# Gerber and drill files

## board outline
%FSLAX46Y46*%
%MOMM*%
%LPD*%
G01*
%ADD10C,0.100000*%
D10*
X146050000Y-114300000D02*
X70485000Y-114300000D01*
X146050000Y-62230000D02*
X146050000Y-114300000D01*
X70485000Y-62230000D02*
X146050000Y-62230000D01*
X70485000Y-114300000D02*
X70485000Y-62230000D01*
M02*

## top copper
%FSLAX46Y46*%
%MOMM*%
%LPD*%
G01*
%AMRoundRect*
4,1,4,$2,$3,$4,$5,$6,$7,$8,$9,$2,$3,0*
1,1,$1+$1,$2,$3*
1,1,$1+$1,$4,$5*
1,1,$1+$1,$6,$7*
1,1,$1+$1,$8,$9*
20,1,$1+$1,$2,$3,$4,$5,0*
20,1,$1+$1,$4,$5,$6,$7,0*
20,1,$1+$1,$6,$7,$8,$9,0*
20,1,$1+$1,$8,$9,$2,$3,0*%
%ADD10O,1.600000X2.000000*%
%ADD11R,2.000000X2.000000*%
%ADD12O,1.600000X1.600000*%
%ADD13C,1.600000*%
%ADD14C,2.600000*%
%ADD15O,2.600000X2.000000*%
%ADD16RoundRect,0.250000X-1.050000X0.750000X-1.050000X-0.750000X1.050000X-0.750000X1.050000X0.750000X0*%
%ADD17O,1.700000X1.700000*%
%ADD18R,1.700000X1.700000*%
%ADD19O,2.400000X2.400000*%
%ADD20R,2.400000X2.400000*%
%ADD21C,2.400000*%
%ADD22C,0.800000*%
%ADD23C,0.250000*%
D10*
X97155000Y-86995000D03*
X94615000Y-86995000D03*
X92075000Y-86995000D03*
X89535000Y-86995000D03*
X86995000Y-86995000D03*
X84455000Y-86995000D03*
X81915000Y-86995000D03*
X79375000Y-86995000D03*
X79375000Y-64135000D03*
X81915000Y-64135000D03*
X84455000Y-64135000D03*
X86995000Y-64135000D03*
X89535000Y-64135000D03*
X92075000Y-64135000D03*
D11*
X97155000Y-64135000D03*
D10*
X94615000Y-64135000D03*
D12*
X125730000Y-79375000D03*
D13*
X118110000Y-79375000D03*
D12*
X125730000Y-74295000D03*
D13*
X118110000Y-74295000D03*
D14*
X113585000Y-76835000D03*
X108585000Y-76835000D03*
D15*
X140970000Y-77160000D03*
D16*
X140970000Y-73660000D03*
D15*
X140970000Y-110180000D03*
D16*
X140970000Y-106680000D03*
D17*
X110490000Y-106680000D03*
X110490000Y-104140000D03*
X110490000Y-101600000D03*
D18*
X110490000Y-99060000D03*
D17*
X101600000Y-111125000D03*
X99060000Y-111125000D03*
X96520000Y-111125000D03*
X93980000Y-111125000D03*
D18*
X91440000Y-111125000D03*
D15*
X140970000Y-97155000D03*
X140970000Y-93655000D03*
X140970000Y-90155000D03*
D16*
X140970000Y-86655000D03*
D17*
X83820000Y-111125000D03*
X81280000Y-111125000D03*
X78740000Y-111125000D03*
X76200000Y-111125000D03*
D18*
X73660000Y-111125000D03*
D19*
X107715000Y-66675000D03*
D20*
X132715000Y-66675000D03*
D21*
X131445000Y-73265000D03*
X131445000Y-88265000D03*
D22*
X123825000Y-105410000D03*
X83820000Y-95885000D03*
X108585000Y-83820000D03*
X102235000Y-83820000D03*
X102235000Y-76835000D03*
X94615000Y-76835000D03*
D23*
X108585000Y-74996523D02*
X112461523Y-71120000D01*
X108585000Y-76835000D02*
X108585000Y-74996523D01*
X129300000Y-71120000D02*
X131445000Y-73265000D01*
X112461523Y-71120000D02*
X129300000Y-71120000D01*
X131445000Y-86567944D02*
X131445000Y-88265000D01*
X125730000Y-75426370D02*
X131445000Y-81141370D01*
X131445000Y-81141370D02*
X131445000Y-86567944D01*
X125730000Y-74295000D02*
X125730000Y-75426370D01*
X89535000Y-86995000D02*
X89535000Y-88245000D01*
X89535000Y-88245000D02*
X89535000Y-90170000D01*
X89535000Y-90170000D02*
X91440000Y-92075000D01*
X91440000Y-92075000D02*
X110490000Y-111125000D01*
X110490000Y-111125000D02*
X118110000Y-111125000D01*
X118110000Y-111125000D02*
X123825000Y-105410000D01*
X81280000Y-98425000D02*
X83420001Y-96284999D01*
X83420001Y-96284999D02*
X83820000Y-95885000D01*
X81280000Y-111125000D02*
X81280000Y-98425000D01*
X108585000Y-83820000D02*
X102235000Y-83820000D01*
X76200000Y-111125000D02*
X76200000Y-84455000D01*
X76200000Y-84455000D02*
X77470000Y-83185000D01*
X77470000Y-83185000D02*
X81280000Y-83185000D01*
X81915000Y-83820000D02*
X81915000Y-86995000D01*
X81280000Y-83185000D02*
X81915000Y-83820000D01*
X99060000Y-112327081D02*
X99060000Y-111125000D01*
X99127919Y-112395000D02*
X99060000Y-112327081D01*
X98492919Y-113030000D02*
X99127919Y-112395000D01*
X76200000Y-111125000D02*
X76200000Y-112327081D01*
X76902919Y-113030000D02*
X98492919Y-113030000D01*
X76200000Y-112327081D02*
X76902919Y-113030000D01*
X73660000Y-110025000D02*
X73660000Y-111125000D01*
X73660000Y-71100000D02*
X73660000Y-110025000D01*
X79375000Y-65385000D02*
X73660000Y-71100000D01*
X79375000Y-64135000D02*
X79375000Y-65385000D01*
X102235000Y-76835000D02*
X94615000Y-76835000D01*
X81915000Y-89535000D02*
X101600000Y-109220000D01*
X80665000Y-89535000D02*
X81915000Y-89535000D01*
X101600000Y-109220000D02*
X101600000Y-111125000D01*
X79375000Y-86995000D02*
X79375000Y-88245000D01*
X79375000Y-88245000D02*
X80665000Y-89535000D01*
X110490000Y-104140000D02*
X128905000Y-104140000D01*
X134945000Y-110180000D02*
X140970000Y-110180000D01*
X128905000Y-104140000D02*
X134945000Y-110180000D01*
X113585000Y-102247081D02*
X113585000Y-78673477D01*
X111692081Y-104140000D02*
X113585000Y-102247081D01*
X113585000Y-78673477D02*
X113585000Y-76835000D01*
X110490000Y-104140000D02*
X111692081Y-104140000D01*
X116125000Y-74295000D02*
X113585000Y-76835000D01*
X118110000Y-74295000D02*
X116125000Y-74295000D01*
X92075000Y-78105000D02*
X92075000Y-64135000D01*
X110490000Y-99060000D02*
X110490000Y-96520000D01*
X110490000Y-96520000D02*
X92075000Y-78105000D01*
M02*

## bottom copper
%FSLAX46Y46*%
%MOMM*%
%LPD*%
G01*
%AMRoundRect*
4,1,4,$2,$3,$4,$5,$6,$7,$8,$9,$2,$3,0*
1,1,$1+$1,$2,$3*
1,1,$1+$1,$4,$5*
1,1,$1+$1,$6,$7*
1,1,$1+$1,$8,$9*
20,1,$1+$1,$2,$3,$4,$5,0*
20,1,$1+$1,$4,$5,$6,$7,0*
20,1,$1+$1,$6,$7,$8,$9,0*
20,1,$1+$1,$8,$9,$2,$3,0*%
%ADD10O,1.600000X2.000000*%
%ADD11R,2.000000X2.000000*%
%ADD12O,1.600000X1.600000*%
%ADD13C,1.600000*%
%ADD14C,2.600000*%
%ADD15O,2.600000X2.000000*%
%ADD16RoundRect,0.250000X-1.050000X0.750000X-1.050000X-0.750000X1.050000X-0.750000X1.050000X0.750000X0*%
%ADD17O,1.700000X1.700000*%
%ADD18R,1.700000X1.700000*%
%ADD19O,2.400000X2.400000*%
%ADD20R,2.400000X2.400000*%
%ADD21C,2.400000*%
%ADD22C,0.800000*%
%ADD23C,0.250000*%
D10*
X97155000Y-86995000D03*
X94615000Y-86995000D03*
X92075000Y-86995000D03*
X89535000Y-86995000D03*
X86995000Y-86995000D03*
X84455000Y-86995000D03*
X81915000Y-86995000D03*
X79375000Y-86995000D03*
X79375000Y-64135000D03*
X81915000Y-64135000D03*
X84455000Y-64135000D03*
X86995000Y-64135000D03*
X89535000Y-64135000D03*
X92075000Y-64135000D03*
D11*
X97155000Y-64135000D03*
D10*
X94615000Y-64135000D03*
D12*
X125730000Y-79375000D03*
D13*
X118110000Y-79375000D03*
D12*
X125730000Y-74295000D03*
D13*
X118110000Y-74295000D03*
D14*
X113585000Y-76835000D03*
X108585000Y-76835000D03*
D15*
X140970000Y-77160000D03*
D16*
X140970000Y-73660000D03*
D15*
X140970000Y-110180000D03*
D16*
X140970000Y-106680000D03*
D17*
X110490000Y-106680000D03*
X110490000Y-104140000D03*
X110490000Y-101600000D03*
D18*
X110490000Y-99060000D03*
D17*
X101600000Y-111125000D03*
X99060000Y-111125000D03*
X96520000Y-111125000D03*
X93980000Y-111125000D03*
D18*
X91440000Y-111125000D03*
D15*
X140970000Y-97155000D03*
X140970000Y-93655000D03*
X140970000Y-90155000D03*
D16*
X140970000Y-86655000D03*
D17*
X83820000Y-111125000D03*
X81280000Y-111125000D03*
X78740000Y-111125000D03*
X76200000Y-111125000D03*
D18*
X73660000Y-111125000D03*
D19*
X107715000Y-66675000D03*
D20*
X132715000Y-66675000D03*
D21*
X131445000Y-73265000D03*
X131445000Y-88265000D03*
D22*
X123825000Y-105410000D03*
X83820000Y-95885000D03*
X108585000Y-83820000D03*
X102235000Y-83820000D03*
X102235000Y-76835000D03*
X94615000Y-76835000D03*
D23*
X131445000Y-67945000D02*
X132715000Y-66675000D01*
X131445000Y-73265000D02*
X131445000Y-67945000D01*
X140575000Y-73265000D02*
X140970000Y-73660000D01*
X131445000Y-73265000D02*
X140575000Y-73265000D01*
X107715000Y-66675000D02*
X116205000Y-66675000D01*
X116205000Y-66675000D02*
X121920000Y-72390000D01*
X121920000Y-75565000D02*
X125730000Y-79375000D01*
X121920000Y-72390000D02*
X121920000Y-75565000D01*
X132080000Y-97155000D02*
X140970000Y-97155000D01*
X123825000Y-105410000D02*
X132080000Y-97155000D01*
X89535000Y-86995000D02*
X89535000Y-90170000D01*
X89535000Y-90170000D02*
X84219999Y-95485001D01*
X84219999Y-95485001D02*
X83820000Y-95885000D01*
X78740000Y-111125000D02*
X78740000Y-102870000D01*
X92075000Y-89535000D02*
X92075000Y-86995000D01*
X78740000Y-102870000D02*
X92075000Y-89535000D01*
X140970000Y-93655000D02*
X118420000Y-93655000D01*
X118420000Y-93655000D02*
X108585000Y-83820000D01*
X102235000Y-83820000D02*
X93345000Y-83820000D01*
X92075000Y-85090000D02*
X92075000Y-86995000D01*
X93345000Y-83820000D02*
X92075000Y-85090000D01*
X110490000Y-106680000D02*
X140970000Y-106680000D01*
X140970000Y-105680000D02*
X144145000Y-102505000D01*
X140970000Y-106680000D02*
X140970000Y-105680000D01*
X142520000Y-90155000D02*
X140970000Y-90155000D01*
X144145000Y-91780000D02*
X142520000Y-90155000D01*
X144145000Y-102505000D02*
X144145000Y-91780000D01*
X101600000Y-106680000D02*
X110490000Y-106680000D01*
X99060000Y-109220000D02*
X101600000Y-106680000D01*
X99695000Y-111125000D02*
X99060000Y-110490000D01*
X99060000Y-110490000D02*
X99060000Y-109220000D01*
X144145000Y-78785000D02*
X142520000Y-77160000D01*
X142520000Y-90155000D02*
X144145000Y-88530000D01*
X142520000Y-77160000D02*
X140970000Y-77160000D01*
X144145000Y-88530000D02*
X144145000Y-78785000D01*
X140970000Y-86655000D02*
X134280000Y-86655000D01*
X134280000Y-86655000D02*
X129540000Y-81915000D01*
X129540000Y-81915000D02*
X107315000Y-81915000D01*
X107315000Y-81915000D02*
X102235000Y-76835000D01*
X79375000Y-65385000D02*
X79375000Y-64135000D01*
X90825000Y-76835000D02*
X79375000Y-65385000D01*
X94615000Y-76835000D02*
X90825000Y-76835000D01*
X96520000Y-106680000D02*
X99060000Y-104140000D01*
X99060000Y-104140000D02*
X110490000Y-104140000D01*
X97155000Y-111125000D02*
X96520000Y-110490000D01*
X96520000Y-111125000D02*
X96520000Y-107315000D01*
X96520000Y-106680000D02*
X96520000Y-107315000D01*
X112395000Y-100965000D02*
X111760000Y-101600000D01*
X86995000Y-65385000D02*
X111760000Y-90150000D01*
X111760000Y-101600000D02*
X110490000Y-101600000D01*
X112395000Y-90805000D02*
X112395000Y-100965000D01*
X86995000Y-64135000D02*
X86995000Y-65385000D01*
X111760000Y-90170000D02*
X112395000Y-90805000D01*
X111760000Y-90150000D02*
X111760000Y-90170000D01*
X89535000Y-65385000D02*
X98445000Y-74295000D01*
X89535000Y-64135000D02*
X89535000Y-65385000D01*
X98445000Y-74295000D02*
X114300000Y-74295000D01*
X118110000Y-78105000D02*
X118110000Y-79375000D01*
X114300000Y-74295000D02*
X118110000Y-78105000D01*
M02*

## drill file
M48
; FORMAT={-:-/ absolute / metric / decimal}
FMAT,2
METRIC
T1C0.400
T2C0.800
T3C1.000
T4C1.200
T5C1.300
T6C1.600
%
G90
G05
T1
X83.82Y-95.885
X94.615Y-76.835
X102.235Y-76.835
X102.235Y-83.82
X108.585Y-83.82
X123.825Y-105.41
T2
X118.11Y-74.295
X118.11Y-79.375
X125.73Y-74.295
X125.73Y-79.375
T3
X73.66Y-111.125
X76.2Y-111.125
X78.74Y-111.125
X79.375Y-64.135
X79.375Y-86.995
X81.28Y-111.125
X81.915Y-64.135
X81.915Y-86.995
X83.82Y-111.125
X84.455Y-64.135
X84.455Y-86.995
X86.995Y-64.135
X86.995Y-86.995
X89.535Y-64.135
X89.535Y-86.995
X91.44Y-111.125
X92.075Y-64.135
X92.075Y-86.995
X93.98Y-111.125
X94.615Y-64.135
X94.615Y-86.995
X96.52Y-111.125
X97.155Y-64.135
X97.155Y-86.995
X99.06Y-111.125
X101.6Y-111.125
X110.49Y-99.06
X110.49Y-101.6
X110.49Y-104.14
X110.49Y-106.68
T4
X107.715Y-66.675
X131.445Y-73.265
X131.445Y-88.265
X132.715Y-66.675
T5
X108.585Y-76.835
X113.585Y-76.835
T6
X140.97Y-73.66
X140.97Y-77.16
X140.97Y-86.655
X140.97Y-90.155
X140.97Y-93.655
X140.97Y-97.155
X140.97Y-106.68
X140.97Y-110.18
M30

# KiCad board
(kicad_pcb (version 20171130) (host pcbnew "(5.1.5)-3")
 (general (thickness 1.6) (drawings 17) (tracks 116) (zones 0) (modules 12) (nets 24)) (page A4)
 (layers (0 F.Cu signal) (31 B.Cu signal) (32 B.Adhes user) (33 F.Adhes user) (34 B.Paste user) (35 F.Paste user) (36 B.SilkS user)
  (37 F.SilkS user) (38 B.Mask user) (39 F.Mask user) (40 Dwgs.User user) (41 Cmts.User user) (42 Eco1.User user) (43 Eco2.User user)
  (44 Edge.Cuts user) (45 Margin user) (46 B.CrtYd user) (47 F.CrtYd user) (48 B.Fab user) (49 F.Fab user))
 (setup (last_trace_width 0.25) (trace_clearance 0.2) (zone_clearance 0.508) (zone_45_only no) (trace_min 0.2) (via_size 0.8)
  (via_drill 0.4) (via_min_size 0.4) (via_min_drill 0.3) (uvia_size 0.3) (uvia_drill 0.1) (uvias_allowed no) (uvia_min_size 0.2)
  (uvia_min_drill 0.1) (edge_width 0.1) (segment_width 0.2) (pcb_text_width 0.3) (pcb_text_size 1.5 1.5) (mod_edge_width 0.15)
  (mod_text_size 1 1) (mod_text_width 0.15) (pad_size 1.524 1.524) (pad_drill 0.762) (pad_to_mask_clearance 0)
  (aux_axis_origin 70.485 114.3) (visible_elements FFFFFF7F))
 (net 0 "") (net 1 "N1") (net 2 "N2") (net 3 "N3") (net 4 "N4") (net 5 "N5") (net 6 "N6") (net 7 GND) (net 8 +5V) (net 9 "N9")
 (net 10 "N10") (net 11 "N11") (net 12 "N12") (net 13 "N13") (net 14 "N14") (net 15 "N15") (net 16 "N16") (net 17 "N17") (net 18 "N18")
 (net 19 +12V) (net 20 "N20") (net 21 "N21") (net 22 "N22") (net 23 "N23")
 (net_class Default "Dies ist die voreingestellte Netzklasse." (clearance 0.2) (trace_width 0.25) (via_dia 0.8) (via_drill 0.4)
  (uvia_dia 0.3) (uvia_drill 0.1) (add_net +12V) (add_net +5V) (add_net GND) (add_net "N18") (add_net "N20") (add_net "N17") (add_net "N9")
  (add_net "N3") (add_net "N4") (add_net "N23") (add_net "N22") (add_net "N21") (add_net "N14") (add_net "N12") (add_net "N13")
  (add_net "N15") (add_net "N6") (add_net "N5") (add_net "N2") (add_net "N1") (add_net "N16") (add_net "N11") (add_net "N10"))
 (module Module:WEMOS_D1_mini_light (layer F.Cu) (at 97.155 64.135 270)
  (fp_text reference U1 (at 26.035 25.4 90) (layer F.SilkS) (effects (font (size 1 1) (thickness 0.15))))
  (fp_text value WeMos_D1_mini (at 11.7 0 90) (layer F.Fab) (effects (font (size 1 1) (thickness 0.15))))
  (pad 16 thru_hole oval (at 22.86 0 270) (size 2 1.6) (drill 1) (layers *.Cu *.Mask) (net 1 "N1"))
  (pad 15 thru_hole oval (at 22.86 2.54 270) (size 2 1.6) (drill 1) (layers *.Cu *.Mask) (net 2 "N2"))
  (pad 14 thru_hole oval (at 22.86 5.08 270) (size 2 1.6) (drill 1) (layers *.Cu *.Mask) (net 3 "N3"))
  (pad 13 thru_hole oval (at 22.86 7.62 270) (size 2 1.6) (drill 1) (layers *.Cu *.Mask) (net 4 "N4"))
  (pad 12 thru_hole oval (at 22.86 10.16 270) (size 2 1.6) (drill 1) (layers *.Cu *.Mask) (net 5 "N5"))
  (pad 11 thru_hole oval (at 22.86 12.7 270) (size 2 1.6) (drill 1) (layers *.Cu *.Mask) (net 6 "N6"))
  (pad 10 thru_hole oval (at 22.86 15.24 270) (size 2 1.6) (drill 1) (layers *.Cu *.Mask) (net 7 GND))
  (pad 9 thru_hole oval (at 22.86 17.78 270) (size 2 1.6) (drill 1) (layers *.Cu *.Mask) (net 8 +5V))
  (pad 8 thru_hole oval (at 0 17.78 270) (size 2 1.6) (drill 1) (layers *.Cu *.Mask) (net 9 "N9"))
  (pad 7 thru_hole oval (at 0 15.24 270) (size 2 1.6) (drill 1) (layers *.Cu *.Mask) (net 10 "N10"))
  (pad 6 thru_hole oval (at 0 12.7 270) (size 2 1.6) (drill 1) (layers *.Cu *.Mask) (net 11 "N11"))
  (pad 5 thru_hole oval (at 0 10.16 270) (size 2 1.6) (drill 1) (layers *.Cu *.Mask) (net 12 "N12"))
  (pad 4 thru_hole oval (at 0 7.62 270) (size 2 1.6) (drill 1) (layers *.Cu *.Mask) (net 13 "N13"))
  (pad 3 thru_hole oval (at 0 5.08 270) (size 2 1.6) (drill 1) (layers *.Cu *.Mask) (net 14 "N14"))
  (pad 1 thru_hole rect (at 0 0 270) (size 2 2) (drill 1) (layers *.Cu *.Mask) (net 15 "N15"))
  (pad 2 thru_hole oval (at 0 2.54 270) (size 2 1.6) (drill 1) (layers *.Cu *.Mask) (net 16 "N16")))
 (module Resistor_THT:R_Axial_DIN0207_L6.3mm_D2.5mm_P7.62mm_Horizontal (layer F.Cu) (at 118.11 79.375)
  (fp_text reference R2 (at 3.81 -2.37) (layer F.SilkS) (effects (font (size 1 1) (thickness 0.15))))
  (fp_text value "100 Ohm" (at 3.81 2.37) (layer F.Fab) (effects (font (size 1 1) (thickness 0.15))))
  (pad 2 thru_hole oval (at 7.62 0) (size 1.6 1.6) (drill 0.8) (layers *.Cu *.Mask) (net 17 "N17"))
  (pad 1 thru_hole circle (at 0 0) (size 1.6 1.6) (drill 0.8) (layers *.Cu *.Mask) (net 13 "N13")))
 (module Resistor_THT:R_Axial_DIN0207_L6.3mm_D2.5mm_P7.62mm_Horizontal (layer F.Cu) (at 118.11 74.295)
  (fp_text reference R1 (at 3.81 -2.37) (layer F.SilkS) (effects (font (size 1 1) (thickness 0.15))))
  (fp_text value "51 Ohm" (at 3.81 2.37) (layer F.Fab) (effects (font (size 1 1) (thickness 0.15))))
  (pad 2 thru_hole oval (at 7.62 0) (size 1.6 1.6) (drill 0.8) (layers *.Cu *.Mask) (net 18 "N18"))
  (pad 1 thru_hole circle (at 0 0) (size 1.6 1.6) (drill 0.8) (layers *.Cu *.Mask) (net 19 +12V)))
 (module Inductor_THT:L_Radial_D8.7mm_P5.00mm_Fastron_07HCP (layer F.Cu) (at 108.585 76.835)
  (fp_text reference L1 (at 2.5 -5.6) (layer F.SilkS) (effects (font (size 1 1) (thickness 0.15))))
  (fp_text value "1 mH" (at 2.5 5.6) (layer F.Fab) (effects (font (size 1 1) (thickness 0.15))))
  (pad 2 thru_hole circle (at 5 0) (size 2.6 2.6) (drill 1.3) (layers *.Cu *.Mask) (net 19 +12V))
  (pad 1 thru_hole circle (at 0 0) (size 2.6 2.6) (drill 1.3) (layers *.Cu *.Mask) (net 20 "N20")))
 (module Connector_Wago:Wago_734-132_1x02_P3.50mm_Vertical (layer F.Cu) (at 140.97 73.66 270)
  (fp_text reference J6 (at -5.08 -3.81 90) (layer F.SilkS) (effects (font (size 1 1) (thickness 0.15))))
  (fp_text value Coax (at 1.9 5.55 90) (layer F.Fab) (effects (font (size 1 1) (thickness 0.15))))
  (pad 2 thru_hole oval (at 3.5 0 270) (size 2 2.6) (drill 1.6) (layers *.Cu *.Mask) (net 7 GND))
  (pad 1 thru_hole roundrect (at 0 0 270) (size 2 2.6) (drill 1.6) (layers *.Cu *.Mask) (roundrect_rratio 0.125) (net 20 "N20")))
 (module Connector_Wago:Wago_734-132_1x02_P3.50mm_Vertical (layer F.Cu) (at 140.97 106.68 270)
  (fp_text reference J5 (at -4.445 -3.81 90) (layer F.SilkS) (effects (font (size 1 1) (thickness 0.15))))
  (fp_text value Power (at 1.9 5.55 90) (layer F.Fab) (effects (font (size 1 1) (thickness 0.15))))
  (pad 2 thru_hole oval (at 3.5 0 270) (size 2 2.6) (drill 1.6) (layers *.Cu *.Mask) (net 19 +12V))
  (pad 1 thru_hole roundrect (at 0 0 270) (size 2 2.6) (drill 1.6) (layers *.Cu *.Mask) (roundrect_rratio 0.125) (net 7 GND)))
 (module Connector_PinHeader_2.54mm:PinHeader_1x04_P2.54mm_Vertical (layer F.Cu) (at 110.49 99.06)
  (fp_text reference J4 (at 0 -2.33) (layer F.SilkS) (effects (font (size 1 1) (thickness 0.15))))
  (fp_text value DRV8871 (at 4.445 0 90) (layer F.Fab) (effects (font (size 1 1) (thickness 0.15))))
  (pad 4 thru_hole oval (at 0 7.62) (size 1.7 1.7) (drill 1) (layers *.Cu *.Mask) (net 7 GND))
  (pad 3 thru_hole oval (at 0 5.08) (size 1.7 1.7) (drill 1) (layers *.Cu *.Mask) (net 19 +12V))
  (pad 2 thru_hole oval (at 0 2.54) (size 1.7 1.7) (drill 1) (layers *.Cu *.Mask) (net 12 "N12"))
  (pad 1 thru_hole rect (at 0 0) (size 1.7 1.7) (drill 1) (layers *.Cu *.Mask) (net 14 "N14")))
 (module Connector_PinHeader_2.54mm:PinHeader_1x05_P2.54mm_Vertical (layer F.Cu) (at 91.44 111.125 90)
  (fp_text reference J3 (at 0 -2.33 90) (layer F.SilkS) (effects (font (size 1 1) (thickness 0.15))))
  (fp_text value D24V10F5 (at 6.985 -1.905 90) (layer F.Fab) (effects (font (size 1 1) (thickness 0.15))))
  (pad 5 thru_hole oval (at 0 10.16 90) (size 1.7 1.7) (drill 1) (layers *.Cu *.Mask) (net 8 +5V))
  (pad 4 thru_hole oval (at 0 7.62 90) (size 1.7 1.7) (drill 1) (layers *.Cu *.Mask) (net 7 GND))
  (pad 3 thru_hole oval (at 0 5.08 90) (size 1.7 1.7) (drill 1) (layers *.Cu *.Mask) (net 19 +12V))
  (pad 2 thru_hole oval (at 0 2.54 90) (size 1.7 1.7) (drill 1) (layers *.Cu *.Mask) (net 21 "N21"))
  (pad 1 thru_hole rect (at 0 0 90) (size 1.7 1.7) (drill 1) (layers *.Cu *.Mask) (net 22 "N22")))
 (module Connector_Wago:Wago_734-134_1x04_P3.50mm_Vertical (layer F.Cu) (at 140.97 86.655 270)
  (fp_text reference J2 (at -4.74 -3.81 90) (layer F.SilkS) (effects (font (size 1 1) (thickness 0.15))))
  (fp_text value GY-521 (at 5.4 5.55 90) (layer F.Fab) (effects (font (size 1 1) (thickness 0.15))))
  (pad 4 thru_hole oval (at 10.5 0 270) (size 2 2.6) (drill 1.6) (layers *.Cu *.Mask) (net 4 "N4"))
  (pad 3 thru_hole oval (at 7 0 270) (size 2 2.6) (drill 1.6) (layers *.Cu *.Mask) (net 3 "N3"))
  (pad 2 thru_hole oval (at 3.5 0 270) (size 2 2.6) (drill 1.6) (layers *.Cu *.Mask) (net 7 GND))
  (pad 1 thru_hole roundrect (at 0 0 270) (size 2 2.6) (drill 1.6) (layers *.Cu *.Mask) (roundrect_rratio 0.125) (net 9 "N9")))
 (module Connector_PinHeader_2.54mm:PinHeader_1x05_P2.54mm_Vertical (layer F.Cu) (at 73.66 111.125 90)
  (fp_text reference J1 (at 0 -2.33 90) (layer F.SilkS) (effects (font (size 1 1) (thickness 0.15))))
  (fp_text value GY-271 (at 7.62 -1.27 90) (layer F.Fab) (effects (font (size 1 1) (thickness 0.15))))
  (pad 5 thru_hole oval (at 0 10.16 90) (size 1.7 1.7) (drill 1) (layers *.Cu *.Mask) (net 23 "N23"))
  (pad 4 thru_hole oval (at 0 7.62 90) (size 1.7 1.7) (drill 1) (layers *.Cu *.Mask) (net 4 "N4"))
  (pad 3 thru_hole oval (at 0 5.08 90) (size 1.7 1.7) (drill 1) (layers *.Cu *.Mask) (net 3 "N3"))
  (pad 2 thru_hole oval (at 0 2.54 90) (size 1.7 1.7) (drill 1) (layers *.Cu *.Mask) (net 7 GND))
  (pad 1 thru_hole rect (at 0 0 90) (size 1.7 1.7) (drill 1) (layers *.Cu *.Mask) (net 9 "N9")))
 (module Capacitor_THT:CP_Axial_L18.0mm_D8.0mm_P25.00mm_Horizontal (layer F.Cu) (at 132.715 66.675 180)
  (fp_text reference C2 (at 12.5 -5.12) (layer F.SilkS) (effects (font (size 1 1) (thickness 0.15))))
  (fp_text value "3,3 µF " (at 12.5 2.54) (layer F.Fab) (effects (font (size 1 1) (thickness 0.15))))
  (pad 2 thru_hole oval (at 25 0 180) (size 2.4 2.4) (drill 1.2) (layers *.Cu *.Mask) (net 17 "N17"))
  (pad 1 thru_hole rect (at 0 0 180) (size 2.4 2.4) (drill 1.2) (layers *.Cu *.Mask) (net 20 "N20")))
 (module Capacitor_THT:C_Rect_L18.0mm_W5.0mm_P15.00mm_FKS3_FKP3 (layer F.Cu) (at 131.445 88.265 90)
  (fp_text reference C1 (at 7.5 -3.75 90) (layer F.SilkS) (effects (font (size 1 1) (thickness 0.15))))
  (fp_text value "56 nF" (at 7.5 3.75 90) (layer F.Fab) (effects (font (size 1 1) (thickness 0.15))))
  (pad 2 thru_hole circle (at 15 0 90) (size 2.4 2.4) (drill 1.2) (layers *.Cu *.Mask) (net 20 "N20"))
  (pad 1 thru_hole circle (at 0 0 90) (size 2.4 2.4) (drill 1.2) (layers *.Cu *.Mask) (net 18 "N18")))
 (gr_line (start 146.05 114.3) (end 70.485 114.3) (layer Edge.Cuts) (width 0.1))
 (gr_line (start 146.05 62.23) (end 146.05 114.3) (layer Edge.Cuts) (width 0.1))
 (gr_line (start 70.485 62.23) (end 146.05 62.23) (layer Edge.Cuts) (width 0.1))
 (gr_line (start 70.485 114.3) (end 70.485 62.23) (layer Edge.Cuts) (width 0.1))
 (segment (start 131.445 67.945) (end 132.715 66.675) (width 0.25) (layer B.Cu) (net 20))
 (segment (start 131.445 73.265) (end 131.445 67.945) (width 0.25) (layer B.Cu) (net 20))
 (segment (start 140.575 73.265) (end 140.97 73.66) (width 0.25) (layer B.Cu) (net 20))
 (segment (start 131.445 73.265) (end 140.575 73.265) (width 0.25) (layer B.Cu) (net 20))
 (segment (start 108.585 74.996523) (end 112.461523 71.12) (width 0.25) (layer F.Cu) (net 20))
 (segment (start 108.585 76.835) (end 108.585 74.996523) (width 0.25) (layer F.Cu) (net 20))
 (segment (start 129.3 71.12) (end 131.445 73.265) (width 0.25) (layer F.Cu) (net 20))
 (segment (start 112.461523 71.12) (end 129.3 71.12) (width 0.25) (layer F.Cu) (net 20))
 (segment (start 131.445 86.567944) (end 131.445 88.265) (width 0.25) (layer F.Cu) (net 18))
 (segment (start 125.73 75.42637) (end 131.445 81.14137) (width 0.25) (layer F.Cu) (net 18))
 (segment (start 131.445 81.14137) (end 131.445 86.567944) (width 0.25) (layer F.Cu) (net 18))
 (segment (start 125.73 74.295) (end 125.73 75.42637) (width 0.25) (layer F.Cu) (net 18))
 (segment (start 107.715 66.675) (end 116.205 66.675) (width 0.25) (layer B.Cu) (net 17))
 (segment (start 116.205 66.675) (end 121.92 72.39) (width 0.25) (layer B.Cu) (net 17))
 (segment (start 121.92 75.565) (end 125.73 79.375) (width 0.25) (layer B.Cu) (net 17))
 (segment (start 121.92 72.39) (end 121.92 75.565) (width 0.25) (layer B.Cu) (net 17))
 (segment (start 89.535 86.995) (end 89.535 88.245) (width 0.25) (layer F.Cu) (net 4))
 (segment (start 89.535 88.245) (end 89.535 90.17) (width 0.25) (layer F.Cu) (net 4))
 (segment (start 89.535 90.17) (end 91.44 92.075) (width 0.25) (layer F.Cu) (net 4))
 (segment (start 91.44 92.075) (end 110.49 111.125) (width 0.25) (layer F.Cu) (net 4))
 (via (at 123.825 105.41) (size 0.8) (drill 0.4) (layers F.Cu B.Cu) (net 4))
 (segment (start 110.49 111.125) (end 118.11 111.125) (width 0.25) (layer F.Cu) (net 4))
 (segment (start 118.11 111.125) (end 123.825 105.41) (width 0.25) (layer F.Cu) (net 4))
 (segment (start 132.08 97.155) (end 140.97 97.155) (width 0.25) (layer B.Cu) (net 4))
 (segment (start 123.825 105.41) (end 132.08 97.155) (width 0.25) (layer B.Cu) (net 4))
 (via (at 83.82 95.885) (size 0.8) (drill 0.4) (layers F.Cu B.Cu) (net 4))
 (segment (start 81.28 98.425) (end 83.420001 96.284999) (width 0.25) (layer F.Cu) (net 4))
 (segment (start 89.535 86.995) (end 89.535 90.17) (width 0.25) (layer B.Cu) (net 4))
 (segment (start 83.420001 96.284999) (end 83.82 95.885) (width 0.25) (layer F.Cu) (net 4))
 (segment (start 81.28 111.125) (end 81.28 98.425) (width 0.25) (layer F.Cu) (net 4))
 (segment (start 89.535 90.17) (end 84.219999 95.485001) (width 0.25) (layer B.Cu) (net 4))
 (segment (start 84.219999 95.485001) (end 83.82 95.885) (width 0.25) (layer B.Cu) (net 4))
 (segment (start 78.74 111.125) (end 78.74 102.87) (width 0.25) (layer B.Cu) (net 3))
 (segment (start 92.075 89.535) (end 92.075 86.995) (width 0.25) (layer B.Cu) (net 3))
 (segment (start 78.74 102.87) (end 92.075 89.535) (width 0.25) (layer B.Cu) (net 3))
 (segment (start 140.97 93.655) (end 118.42 93.655) (width 0.25) (layer B.Cu) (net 3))
 (via (at 108.585 83.82) (size 0.8) (drill 0.4) (layers F.Cu B.Cu) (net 3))
 (segment (start 118.42 93.655) (end 108.585 83.82) (width 0.25) (layer B.Cu) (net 3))
 (segment (start 108.585 83.82) (end 102.235 83.82) (width 0.25) (layer F.Cu) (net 3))
 (via (at 102.235 83.82) (size 0.8) (drill 0.4) (layers F.Cu B.Cu) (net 3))
 (segment (start 102.235 83.82) (end 93.345 83.82) (width 0.25) (layer B.Cu) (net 3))
 (segment (start 92.075 85.09) (end 92.075 86.995) (width 0.25) (layer B.Cu) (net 3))
 (segment (start 93.345 83.82) (end 92.075 85.09) (width 0.25) (layer B.Cu) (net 3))
 (segment (start 76.2 111.125) (end 76.2 84.455) (width 0.25) (layer F.Cu) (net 7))
 (segment (start 76.2 84.455) (end 77.47 83.185) (width 0.25) (layer F.Cu) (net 7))
 (segment (start 77.47 83.185) (end 81.28 83.185) (width 0.25) (layer F.Cu) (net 7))
 (segment (start 81.915 83.82) (end 81.915 86.995) (width 0.25) (layer F.Cu) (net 7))
 (segment (start 81.28 83.185) (end 81.915 83.82) (width 0.25) (layer F.Cu) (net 7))
 (segment (start 110.49 106.68) (end 140.97 106.68) (width 0.25) (layer B.Cu) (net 7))
 (segment (start 140.97 105.68) (end 144.145 102.505) (width 0.25) (layer B.Cu) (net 7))
 (segment (start 140.97 106.68) (end 140.97 105.68) (width 0.25) (layer B.Cu) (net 7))
 (segment (start 142.52 90.155) (end 140.97 90.155) (width 0.25) (layer B.Cu) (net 7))
 (segment (start 144.145 91.78) (end 142.52 90.155) (width 0.25) (layer B.Cu) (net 7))
 (segment (start 144.145 102.505) (end 144.145 91.78) (width 0.25) (layer B.Cu) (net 7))
 (segment (start 101.6 106.68) (end 110.49 106.68) (width 0.25) (layer B.Cu) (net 7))
 (segment (start 99.06 109.22) (end 101.6 106.68) (width 0.25) (layer B.Cu) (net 7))
 (segment (start 99.695 111.125) (end 99.06 110.49) (width 0.25) (layer B.Cu) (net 7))
 (segment (start 99.06 110.49) (end 99.06 109.22) (width 0.25) (layer B.Cu) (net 7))
 (segment (start 99.06 112.327081) (end 99.06 111.125) (width 0.25) (layer F.Cu) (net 7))
 (segment (start 99.127919 112.395) (end 99.06 112.327081) (width 0.25) (layer F.Cu) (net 7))
 (segment (start 98.492919 113.03) (end 99.127919 112.395) (width 0.25) (layer F.Cu) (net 7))
 (segment (start 76.2 111.125) (end 76.2 112.327081) (width 0.25) (layer F.Cu) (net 7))
 (segment (start 76.902919 113.03) (end 98.492919 113.03) (width 0.25) (layer F.Cu) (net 7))
 (segment (start 76.2 112.327081) (end 76.902919 113.03) (width 0.25) (layer F.Cu) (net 7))
 (segment (start 144.145 78.785) (end 142.52 77.16) (width 0.25) (layer B.Cu) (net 7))
 (segment (start 142.52 90.155) (end 144.145 88.53) (width 0.25) (layer B.Cu) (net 7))
 (segment (start 142.52 77.16) (end 140.97 77.16) (width 0.25) (layer B.Cu) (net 7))
 (segment (start 144.145 88.53) (end 144.145 78.785) (width 0.25) (layer B.Cu) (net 7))
 (segment (start 73.66 110.025) (end 73.66 111.125) (width 0.25) (layer F.Cu) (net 9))
 (segment (start 73.66 71.1) (end 73.66 110.025) (width 0.25) (layer F.Cu) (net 9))
 (segment (start 79.375 65.385) (end 73.66 71.1) (width 0.25) (layer F.Cu) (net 9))
 (segment (start 79.375 64.135) (end 79.375 65.385) (width 0.25) (layer F.Cu) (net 9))
 (segment (start 140.97 86.655) (end 134.28 86.655) (width 0.25) (layer B.Cu) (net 9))
 (segment (start 134.28 86.655) (end 129.54 81.915) (width 0.25) (layer B.Cu) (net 9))
 (segment (start 129.54 81.915) (end 107.315 81.915) (width 0.25) (layer B.Cu) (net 9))
 (via (at 102.235 76.835) (size 0.8) (drill 0.4) (layers F.Cu B.Cu) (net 9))
 (segment (start 107.315 81.915) (end 102.235 76.835) (width 0.25) (layer B.Cu) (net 9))
 (segment (start 102.235 76.835) (end 94.615 76.835) (width 0.25) (layer F.Cu) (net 9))
 (via (at 94.615 76.835) (size 0.8) (drill 0.4) (layers F.Cu B.Cu) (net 9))
 (segment (start 79.375 65.385) (end 79.375 64.135) (width 0.25) (layer B.Cu) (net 9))
 (segment (start 90.825 76.835) (end 79.375 65.385) (width 0.25) (layer B.Cu) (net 9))
 (segment (start 94.615 76.835) (end 90.825 76.835) (width 0.25) (layer B.Cu) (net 9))
 (segment (start 81.915 89.535) (end 101.6 109.22) (width 0.25) (layer F.Cu) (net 8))
 (segment (start 80.665 89.535) (end 81.915 89.535) (width 0.25) (layer F.Cu) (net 8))
 (segment (start 101.6 109.22) (end 101.6 111.125) (width 0.25) (layer F.Cu) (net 8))
 (segment (start 79.375 86.995) (end 79.375 88.245) (width 0.25) (layer F.Cu) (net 8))
 (segment (start 79.375 88.245) (end 80.665 89.535) (width 0.25) (layer F.Cu) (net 8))
 (segment (start 110.49 104.14) (end 128.905 104.14) (width 0.25) (layer F.Cu) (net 19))
 (segment (start 134.945 110.18) (end 140.97 110.18) (width 0.25) (layer F.Cu) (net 19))
 (segment (start 128.905 104.14) (end 134.945 110.18) (width 0.25) (layer F.Cu) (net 19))
 (segment (start 113.585 102.247081) (end 113.585 78.673477) (width 0.25) (layer F.Cu) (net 19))
 (segment (start 111.692081 104.14) (end 113.585 102.247081) (width 0.25) (layer F.Cu) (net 19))
 (segment (start 113.585 78.673477) (end 113.585 76.835) (width 0.25) (layer F.Cu) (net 19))
 (segment (start 110.49 104.14) (end 111.692081 104.14) (width 0.25) (layer F.Cu) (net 19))
 (segment (start 116.125 74.295) (end 113.585 76.835) (width 0.25) (layer F.Cu) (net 19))
 (segment (start 118.11 74.295) (end 116.125 74.295) (width 0.25) (layer F.Cu) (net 19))
 (segment (start 96.52 106.68) (end 99.06 104.14) (width 0.25) (layer B.Cu) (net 19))
 (segment (start 99.06 104.14) (end 110.49 104.14) (width 0.25) (layer B.Cu) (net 19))
 (segment (start 97.155 111.125) (end 96.52 110.49) (width 0.25) (layer B.Cu) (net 19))
 (segment (start 96.52 111.125) (end 96.52 107.315) (width 0.25) (layer B.Cu) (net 19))
 (segment (start 96.52 106.68) (end 96.52 107.315) (width 0.25) (layer B.Cu) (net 19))
 (segment (start 112.395 100.965) (end 111.76 101.6) (width 0.25) (layer B.Cu) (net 12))
 (segment (start 86.995 65.385) (end 111.76 90.15) (width 0.25) (layer B.Cu) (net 12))
 (segment (start 111.76 101.6) (end 110.49 101.6) (width 0.25) (layer B.Cu) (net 12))
 (segment (start 112.395 90.805) (end 112.395 100.965) (width 0.25) (layer B.Cu) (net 12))
 (segment (start 86.995 64.135) (end 86.995 65.385) (width 0.25) (layer B.Cu) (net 12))
 (segment (start 111.76 90.17) (end 112.395 90.805) (width 0.25) (layer B.Cu) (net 12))
 (segment (start 111.76 90.15) (end 111.76 90.17) (width 0.25) (layer B.Cu) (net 12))
 (segment (start 92.075 78.105) (end 92.075 64.135) (width 0.25) (layer F.Cu) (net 14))
 (segment (start 110.49 99.06) (end 110.49 96.52) (width 0.25) (layer F.Cu) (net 14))
 (segment (start 110.49 96.52) (end 92.075 78.105) (width 0.25) (layer F.Cu) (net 14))
 (segment (start 89.535 65.385) (end 98.445 74.295) (width 0.25) (layer B.Cu) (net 13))
 (segment (start 89.535 64.135) (end 89.535 65.385) (width 0.25) (layer B.Cu) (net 13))
 (segment (start 98.445 74.295) (end 114.3 74.295) (width 0.25) (layer B.Cu) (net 13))
 (segment (start 118.11 78.105) (end 118.11 79.375) (width 0.25) (layer B.Cu) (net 13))
 (segment (start 114.3 74.295) (end 118.11 78.105) (width 0.25) (layer B.Cu) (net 13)))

